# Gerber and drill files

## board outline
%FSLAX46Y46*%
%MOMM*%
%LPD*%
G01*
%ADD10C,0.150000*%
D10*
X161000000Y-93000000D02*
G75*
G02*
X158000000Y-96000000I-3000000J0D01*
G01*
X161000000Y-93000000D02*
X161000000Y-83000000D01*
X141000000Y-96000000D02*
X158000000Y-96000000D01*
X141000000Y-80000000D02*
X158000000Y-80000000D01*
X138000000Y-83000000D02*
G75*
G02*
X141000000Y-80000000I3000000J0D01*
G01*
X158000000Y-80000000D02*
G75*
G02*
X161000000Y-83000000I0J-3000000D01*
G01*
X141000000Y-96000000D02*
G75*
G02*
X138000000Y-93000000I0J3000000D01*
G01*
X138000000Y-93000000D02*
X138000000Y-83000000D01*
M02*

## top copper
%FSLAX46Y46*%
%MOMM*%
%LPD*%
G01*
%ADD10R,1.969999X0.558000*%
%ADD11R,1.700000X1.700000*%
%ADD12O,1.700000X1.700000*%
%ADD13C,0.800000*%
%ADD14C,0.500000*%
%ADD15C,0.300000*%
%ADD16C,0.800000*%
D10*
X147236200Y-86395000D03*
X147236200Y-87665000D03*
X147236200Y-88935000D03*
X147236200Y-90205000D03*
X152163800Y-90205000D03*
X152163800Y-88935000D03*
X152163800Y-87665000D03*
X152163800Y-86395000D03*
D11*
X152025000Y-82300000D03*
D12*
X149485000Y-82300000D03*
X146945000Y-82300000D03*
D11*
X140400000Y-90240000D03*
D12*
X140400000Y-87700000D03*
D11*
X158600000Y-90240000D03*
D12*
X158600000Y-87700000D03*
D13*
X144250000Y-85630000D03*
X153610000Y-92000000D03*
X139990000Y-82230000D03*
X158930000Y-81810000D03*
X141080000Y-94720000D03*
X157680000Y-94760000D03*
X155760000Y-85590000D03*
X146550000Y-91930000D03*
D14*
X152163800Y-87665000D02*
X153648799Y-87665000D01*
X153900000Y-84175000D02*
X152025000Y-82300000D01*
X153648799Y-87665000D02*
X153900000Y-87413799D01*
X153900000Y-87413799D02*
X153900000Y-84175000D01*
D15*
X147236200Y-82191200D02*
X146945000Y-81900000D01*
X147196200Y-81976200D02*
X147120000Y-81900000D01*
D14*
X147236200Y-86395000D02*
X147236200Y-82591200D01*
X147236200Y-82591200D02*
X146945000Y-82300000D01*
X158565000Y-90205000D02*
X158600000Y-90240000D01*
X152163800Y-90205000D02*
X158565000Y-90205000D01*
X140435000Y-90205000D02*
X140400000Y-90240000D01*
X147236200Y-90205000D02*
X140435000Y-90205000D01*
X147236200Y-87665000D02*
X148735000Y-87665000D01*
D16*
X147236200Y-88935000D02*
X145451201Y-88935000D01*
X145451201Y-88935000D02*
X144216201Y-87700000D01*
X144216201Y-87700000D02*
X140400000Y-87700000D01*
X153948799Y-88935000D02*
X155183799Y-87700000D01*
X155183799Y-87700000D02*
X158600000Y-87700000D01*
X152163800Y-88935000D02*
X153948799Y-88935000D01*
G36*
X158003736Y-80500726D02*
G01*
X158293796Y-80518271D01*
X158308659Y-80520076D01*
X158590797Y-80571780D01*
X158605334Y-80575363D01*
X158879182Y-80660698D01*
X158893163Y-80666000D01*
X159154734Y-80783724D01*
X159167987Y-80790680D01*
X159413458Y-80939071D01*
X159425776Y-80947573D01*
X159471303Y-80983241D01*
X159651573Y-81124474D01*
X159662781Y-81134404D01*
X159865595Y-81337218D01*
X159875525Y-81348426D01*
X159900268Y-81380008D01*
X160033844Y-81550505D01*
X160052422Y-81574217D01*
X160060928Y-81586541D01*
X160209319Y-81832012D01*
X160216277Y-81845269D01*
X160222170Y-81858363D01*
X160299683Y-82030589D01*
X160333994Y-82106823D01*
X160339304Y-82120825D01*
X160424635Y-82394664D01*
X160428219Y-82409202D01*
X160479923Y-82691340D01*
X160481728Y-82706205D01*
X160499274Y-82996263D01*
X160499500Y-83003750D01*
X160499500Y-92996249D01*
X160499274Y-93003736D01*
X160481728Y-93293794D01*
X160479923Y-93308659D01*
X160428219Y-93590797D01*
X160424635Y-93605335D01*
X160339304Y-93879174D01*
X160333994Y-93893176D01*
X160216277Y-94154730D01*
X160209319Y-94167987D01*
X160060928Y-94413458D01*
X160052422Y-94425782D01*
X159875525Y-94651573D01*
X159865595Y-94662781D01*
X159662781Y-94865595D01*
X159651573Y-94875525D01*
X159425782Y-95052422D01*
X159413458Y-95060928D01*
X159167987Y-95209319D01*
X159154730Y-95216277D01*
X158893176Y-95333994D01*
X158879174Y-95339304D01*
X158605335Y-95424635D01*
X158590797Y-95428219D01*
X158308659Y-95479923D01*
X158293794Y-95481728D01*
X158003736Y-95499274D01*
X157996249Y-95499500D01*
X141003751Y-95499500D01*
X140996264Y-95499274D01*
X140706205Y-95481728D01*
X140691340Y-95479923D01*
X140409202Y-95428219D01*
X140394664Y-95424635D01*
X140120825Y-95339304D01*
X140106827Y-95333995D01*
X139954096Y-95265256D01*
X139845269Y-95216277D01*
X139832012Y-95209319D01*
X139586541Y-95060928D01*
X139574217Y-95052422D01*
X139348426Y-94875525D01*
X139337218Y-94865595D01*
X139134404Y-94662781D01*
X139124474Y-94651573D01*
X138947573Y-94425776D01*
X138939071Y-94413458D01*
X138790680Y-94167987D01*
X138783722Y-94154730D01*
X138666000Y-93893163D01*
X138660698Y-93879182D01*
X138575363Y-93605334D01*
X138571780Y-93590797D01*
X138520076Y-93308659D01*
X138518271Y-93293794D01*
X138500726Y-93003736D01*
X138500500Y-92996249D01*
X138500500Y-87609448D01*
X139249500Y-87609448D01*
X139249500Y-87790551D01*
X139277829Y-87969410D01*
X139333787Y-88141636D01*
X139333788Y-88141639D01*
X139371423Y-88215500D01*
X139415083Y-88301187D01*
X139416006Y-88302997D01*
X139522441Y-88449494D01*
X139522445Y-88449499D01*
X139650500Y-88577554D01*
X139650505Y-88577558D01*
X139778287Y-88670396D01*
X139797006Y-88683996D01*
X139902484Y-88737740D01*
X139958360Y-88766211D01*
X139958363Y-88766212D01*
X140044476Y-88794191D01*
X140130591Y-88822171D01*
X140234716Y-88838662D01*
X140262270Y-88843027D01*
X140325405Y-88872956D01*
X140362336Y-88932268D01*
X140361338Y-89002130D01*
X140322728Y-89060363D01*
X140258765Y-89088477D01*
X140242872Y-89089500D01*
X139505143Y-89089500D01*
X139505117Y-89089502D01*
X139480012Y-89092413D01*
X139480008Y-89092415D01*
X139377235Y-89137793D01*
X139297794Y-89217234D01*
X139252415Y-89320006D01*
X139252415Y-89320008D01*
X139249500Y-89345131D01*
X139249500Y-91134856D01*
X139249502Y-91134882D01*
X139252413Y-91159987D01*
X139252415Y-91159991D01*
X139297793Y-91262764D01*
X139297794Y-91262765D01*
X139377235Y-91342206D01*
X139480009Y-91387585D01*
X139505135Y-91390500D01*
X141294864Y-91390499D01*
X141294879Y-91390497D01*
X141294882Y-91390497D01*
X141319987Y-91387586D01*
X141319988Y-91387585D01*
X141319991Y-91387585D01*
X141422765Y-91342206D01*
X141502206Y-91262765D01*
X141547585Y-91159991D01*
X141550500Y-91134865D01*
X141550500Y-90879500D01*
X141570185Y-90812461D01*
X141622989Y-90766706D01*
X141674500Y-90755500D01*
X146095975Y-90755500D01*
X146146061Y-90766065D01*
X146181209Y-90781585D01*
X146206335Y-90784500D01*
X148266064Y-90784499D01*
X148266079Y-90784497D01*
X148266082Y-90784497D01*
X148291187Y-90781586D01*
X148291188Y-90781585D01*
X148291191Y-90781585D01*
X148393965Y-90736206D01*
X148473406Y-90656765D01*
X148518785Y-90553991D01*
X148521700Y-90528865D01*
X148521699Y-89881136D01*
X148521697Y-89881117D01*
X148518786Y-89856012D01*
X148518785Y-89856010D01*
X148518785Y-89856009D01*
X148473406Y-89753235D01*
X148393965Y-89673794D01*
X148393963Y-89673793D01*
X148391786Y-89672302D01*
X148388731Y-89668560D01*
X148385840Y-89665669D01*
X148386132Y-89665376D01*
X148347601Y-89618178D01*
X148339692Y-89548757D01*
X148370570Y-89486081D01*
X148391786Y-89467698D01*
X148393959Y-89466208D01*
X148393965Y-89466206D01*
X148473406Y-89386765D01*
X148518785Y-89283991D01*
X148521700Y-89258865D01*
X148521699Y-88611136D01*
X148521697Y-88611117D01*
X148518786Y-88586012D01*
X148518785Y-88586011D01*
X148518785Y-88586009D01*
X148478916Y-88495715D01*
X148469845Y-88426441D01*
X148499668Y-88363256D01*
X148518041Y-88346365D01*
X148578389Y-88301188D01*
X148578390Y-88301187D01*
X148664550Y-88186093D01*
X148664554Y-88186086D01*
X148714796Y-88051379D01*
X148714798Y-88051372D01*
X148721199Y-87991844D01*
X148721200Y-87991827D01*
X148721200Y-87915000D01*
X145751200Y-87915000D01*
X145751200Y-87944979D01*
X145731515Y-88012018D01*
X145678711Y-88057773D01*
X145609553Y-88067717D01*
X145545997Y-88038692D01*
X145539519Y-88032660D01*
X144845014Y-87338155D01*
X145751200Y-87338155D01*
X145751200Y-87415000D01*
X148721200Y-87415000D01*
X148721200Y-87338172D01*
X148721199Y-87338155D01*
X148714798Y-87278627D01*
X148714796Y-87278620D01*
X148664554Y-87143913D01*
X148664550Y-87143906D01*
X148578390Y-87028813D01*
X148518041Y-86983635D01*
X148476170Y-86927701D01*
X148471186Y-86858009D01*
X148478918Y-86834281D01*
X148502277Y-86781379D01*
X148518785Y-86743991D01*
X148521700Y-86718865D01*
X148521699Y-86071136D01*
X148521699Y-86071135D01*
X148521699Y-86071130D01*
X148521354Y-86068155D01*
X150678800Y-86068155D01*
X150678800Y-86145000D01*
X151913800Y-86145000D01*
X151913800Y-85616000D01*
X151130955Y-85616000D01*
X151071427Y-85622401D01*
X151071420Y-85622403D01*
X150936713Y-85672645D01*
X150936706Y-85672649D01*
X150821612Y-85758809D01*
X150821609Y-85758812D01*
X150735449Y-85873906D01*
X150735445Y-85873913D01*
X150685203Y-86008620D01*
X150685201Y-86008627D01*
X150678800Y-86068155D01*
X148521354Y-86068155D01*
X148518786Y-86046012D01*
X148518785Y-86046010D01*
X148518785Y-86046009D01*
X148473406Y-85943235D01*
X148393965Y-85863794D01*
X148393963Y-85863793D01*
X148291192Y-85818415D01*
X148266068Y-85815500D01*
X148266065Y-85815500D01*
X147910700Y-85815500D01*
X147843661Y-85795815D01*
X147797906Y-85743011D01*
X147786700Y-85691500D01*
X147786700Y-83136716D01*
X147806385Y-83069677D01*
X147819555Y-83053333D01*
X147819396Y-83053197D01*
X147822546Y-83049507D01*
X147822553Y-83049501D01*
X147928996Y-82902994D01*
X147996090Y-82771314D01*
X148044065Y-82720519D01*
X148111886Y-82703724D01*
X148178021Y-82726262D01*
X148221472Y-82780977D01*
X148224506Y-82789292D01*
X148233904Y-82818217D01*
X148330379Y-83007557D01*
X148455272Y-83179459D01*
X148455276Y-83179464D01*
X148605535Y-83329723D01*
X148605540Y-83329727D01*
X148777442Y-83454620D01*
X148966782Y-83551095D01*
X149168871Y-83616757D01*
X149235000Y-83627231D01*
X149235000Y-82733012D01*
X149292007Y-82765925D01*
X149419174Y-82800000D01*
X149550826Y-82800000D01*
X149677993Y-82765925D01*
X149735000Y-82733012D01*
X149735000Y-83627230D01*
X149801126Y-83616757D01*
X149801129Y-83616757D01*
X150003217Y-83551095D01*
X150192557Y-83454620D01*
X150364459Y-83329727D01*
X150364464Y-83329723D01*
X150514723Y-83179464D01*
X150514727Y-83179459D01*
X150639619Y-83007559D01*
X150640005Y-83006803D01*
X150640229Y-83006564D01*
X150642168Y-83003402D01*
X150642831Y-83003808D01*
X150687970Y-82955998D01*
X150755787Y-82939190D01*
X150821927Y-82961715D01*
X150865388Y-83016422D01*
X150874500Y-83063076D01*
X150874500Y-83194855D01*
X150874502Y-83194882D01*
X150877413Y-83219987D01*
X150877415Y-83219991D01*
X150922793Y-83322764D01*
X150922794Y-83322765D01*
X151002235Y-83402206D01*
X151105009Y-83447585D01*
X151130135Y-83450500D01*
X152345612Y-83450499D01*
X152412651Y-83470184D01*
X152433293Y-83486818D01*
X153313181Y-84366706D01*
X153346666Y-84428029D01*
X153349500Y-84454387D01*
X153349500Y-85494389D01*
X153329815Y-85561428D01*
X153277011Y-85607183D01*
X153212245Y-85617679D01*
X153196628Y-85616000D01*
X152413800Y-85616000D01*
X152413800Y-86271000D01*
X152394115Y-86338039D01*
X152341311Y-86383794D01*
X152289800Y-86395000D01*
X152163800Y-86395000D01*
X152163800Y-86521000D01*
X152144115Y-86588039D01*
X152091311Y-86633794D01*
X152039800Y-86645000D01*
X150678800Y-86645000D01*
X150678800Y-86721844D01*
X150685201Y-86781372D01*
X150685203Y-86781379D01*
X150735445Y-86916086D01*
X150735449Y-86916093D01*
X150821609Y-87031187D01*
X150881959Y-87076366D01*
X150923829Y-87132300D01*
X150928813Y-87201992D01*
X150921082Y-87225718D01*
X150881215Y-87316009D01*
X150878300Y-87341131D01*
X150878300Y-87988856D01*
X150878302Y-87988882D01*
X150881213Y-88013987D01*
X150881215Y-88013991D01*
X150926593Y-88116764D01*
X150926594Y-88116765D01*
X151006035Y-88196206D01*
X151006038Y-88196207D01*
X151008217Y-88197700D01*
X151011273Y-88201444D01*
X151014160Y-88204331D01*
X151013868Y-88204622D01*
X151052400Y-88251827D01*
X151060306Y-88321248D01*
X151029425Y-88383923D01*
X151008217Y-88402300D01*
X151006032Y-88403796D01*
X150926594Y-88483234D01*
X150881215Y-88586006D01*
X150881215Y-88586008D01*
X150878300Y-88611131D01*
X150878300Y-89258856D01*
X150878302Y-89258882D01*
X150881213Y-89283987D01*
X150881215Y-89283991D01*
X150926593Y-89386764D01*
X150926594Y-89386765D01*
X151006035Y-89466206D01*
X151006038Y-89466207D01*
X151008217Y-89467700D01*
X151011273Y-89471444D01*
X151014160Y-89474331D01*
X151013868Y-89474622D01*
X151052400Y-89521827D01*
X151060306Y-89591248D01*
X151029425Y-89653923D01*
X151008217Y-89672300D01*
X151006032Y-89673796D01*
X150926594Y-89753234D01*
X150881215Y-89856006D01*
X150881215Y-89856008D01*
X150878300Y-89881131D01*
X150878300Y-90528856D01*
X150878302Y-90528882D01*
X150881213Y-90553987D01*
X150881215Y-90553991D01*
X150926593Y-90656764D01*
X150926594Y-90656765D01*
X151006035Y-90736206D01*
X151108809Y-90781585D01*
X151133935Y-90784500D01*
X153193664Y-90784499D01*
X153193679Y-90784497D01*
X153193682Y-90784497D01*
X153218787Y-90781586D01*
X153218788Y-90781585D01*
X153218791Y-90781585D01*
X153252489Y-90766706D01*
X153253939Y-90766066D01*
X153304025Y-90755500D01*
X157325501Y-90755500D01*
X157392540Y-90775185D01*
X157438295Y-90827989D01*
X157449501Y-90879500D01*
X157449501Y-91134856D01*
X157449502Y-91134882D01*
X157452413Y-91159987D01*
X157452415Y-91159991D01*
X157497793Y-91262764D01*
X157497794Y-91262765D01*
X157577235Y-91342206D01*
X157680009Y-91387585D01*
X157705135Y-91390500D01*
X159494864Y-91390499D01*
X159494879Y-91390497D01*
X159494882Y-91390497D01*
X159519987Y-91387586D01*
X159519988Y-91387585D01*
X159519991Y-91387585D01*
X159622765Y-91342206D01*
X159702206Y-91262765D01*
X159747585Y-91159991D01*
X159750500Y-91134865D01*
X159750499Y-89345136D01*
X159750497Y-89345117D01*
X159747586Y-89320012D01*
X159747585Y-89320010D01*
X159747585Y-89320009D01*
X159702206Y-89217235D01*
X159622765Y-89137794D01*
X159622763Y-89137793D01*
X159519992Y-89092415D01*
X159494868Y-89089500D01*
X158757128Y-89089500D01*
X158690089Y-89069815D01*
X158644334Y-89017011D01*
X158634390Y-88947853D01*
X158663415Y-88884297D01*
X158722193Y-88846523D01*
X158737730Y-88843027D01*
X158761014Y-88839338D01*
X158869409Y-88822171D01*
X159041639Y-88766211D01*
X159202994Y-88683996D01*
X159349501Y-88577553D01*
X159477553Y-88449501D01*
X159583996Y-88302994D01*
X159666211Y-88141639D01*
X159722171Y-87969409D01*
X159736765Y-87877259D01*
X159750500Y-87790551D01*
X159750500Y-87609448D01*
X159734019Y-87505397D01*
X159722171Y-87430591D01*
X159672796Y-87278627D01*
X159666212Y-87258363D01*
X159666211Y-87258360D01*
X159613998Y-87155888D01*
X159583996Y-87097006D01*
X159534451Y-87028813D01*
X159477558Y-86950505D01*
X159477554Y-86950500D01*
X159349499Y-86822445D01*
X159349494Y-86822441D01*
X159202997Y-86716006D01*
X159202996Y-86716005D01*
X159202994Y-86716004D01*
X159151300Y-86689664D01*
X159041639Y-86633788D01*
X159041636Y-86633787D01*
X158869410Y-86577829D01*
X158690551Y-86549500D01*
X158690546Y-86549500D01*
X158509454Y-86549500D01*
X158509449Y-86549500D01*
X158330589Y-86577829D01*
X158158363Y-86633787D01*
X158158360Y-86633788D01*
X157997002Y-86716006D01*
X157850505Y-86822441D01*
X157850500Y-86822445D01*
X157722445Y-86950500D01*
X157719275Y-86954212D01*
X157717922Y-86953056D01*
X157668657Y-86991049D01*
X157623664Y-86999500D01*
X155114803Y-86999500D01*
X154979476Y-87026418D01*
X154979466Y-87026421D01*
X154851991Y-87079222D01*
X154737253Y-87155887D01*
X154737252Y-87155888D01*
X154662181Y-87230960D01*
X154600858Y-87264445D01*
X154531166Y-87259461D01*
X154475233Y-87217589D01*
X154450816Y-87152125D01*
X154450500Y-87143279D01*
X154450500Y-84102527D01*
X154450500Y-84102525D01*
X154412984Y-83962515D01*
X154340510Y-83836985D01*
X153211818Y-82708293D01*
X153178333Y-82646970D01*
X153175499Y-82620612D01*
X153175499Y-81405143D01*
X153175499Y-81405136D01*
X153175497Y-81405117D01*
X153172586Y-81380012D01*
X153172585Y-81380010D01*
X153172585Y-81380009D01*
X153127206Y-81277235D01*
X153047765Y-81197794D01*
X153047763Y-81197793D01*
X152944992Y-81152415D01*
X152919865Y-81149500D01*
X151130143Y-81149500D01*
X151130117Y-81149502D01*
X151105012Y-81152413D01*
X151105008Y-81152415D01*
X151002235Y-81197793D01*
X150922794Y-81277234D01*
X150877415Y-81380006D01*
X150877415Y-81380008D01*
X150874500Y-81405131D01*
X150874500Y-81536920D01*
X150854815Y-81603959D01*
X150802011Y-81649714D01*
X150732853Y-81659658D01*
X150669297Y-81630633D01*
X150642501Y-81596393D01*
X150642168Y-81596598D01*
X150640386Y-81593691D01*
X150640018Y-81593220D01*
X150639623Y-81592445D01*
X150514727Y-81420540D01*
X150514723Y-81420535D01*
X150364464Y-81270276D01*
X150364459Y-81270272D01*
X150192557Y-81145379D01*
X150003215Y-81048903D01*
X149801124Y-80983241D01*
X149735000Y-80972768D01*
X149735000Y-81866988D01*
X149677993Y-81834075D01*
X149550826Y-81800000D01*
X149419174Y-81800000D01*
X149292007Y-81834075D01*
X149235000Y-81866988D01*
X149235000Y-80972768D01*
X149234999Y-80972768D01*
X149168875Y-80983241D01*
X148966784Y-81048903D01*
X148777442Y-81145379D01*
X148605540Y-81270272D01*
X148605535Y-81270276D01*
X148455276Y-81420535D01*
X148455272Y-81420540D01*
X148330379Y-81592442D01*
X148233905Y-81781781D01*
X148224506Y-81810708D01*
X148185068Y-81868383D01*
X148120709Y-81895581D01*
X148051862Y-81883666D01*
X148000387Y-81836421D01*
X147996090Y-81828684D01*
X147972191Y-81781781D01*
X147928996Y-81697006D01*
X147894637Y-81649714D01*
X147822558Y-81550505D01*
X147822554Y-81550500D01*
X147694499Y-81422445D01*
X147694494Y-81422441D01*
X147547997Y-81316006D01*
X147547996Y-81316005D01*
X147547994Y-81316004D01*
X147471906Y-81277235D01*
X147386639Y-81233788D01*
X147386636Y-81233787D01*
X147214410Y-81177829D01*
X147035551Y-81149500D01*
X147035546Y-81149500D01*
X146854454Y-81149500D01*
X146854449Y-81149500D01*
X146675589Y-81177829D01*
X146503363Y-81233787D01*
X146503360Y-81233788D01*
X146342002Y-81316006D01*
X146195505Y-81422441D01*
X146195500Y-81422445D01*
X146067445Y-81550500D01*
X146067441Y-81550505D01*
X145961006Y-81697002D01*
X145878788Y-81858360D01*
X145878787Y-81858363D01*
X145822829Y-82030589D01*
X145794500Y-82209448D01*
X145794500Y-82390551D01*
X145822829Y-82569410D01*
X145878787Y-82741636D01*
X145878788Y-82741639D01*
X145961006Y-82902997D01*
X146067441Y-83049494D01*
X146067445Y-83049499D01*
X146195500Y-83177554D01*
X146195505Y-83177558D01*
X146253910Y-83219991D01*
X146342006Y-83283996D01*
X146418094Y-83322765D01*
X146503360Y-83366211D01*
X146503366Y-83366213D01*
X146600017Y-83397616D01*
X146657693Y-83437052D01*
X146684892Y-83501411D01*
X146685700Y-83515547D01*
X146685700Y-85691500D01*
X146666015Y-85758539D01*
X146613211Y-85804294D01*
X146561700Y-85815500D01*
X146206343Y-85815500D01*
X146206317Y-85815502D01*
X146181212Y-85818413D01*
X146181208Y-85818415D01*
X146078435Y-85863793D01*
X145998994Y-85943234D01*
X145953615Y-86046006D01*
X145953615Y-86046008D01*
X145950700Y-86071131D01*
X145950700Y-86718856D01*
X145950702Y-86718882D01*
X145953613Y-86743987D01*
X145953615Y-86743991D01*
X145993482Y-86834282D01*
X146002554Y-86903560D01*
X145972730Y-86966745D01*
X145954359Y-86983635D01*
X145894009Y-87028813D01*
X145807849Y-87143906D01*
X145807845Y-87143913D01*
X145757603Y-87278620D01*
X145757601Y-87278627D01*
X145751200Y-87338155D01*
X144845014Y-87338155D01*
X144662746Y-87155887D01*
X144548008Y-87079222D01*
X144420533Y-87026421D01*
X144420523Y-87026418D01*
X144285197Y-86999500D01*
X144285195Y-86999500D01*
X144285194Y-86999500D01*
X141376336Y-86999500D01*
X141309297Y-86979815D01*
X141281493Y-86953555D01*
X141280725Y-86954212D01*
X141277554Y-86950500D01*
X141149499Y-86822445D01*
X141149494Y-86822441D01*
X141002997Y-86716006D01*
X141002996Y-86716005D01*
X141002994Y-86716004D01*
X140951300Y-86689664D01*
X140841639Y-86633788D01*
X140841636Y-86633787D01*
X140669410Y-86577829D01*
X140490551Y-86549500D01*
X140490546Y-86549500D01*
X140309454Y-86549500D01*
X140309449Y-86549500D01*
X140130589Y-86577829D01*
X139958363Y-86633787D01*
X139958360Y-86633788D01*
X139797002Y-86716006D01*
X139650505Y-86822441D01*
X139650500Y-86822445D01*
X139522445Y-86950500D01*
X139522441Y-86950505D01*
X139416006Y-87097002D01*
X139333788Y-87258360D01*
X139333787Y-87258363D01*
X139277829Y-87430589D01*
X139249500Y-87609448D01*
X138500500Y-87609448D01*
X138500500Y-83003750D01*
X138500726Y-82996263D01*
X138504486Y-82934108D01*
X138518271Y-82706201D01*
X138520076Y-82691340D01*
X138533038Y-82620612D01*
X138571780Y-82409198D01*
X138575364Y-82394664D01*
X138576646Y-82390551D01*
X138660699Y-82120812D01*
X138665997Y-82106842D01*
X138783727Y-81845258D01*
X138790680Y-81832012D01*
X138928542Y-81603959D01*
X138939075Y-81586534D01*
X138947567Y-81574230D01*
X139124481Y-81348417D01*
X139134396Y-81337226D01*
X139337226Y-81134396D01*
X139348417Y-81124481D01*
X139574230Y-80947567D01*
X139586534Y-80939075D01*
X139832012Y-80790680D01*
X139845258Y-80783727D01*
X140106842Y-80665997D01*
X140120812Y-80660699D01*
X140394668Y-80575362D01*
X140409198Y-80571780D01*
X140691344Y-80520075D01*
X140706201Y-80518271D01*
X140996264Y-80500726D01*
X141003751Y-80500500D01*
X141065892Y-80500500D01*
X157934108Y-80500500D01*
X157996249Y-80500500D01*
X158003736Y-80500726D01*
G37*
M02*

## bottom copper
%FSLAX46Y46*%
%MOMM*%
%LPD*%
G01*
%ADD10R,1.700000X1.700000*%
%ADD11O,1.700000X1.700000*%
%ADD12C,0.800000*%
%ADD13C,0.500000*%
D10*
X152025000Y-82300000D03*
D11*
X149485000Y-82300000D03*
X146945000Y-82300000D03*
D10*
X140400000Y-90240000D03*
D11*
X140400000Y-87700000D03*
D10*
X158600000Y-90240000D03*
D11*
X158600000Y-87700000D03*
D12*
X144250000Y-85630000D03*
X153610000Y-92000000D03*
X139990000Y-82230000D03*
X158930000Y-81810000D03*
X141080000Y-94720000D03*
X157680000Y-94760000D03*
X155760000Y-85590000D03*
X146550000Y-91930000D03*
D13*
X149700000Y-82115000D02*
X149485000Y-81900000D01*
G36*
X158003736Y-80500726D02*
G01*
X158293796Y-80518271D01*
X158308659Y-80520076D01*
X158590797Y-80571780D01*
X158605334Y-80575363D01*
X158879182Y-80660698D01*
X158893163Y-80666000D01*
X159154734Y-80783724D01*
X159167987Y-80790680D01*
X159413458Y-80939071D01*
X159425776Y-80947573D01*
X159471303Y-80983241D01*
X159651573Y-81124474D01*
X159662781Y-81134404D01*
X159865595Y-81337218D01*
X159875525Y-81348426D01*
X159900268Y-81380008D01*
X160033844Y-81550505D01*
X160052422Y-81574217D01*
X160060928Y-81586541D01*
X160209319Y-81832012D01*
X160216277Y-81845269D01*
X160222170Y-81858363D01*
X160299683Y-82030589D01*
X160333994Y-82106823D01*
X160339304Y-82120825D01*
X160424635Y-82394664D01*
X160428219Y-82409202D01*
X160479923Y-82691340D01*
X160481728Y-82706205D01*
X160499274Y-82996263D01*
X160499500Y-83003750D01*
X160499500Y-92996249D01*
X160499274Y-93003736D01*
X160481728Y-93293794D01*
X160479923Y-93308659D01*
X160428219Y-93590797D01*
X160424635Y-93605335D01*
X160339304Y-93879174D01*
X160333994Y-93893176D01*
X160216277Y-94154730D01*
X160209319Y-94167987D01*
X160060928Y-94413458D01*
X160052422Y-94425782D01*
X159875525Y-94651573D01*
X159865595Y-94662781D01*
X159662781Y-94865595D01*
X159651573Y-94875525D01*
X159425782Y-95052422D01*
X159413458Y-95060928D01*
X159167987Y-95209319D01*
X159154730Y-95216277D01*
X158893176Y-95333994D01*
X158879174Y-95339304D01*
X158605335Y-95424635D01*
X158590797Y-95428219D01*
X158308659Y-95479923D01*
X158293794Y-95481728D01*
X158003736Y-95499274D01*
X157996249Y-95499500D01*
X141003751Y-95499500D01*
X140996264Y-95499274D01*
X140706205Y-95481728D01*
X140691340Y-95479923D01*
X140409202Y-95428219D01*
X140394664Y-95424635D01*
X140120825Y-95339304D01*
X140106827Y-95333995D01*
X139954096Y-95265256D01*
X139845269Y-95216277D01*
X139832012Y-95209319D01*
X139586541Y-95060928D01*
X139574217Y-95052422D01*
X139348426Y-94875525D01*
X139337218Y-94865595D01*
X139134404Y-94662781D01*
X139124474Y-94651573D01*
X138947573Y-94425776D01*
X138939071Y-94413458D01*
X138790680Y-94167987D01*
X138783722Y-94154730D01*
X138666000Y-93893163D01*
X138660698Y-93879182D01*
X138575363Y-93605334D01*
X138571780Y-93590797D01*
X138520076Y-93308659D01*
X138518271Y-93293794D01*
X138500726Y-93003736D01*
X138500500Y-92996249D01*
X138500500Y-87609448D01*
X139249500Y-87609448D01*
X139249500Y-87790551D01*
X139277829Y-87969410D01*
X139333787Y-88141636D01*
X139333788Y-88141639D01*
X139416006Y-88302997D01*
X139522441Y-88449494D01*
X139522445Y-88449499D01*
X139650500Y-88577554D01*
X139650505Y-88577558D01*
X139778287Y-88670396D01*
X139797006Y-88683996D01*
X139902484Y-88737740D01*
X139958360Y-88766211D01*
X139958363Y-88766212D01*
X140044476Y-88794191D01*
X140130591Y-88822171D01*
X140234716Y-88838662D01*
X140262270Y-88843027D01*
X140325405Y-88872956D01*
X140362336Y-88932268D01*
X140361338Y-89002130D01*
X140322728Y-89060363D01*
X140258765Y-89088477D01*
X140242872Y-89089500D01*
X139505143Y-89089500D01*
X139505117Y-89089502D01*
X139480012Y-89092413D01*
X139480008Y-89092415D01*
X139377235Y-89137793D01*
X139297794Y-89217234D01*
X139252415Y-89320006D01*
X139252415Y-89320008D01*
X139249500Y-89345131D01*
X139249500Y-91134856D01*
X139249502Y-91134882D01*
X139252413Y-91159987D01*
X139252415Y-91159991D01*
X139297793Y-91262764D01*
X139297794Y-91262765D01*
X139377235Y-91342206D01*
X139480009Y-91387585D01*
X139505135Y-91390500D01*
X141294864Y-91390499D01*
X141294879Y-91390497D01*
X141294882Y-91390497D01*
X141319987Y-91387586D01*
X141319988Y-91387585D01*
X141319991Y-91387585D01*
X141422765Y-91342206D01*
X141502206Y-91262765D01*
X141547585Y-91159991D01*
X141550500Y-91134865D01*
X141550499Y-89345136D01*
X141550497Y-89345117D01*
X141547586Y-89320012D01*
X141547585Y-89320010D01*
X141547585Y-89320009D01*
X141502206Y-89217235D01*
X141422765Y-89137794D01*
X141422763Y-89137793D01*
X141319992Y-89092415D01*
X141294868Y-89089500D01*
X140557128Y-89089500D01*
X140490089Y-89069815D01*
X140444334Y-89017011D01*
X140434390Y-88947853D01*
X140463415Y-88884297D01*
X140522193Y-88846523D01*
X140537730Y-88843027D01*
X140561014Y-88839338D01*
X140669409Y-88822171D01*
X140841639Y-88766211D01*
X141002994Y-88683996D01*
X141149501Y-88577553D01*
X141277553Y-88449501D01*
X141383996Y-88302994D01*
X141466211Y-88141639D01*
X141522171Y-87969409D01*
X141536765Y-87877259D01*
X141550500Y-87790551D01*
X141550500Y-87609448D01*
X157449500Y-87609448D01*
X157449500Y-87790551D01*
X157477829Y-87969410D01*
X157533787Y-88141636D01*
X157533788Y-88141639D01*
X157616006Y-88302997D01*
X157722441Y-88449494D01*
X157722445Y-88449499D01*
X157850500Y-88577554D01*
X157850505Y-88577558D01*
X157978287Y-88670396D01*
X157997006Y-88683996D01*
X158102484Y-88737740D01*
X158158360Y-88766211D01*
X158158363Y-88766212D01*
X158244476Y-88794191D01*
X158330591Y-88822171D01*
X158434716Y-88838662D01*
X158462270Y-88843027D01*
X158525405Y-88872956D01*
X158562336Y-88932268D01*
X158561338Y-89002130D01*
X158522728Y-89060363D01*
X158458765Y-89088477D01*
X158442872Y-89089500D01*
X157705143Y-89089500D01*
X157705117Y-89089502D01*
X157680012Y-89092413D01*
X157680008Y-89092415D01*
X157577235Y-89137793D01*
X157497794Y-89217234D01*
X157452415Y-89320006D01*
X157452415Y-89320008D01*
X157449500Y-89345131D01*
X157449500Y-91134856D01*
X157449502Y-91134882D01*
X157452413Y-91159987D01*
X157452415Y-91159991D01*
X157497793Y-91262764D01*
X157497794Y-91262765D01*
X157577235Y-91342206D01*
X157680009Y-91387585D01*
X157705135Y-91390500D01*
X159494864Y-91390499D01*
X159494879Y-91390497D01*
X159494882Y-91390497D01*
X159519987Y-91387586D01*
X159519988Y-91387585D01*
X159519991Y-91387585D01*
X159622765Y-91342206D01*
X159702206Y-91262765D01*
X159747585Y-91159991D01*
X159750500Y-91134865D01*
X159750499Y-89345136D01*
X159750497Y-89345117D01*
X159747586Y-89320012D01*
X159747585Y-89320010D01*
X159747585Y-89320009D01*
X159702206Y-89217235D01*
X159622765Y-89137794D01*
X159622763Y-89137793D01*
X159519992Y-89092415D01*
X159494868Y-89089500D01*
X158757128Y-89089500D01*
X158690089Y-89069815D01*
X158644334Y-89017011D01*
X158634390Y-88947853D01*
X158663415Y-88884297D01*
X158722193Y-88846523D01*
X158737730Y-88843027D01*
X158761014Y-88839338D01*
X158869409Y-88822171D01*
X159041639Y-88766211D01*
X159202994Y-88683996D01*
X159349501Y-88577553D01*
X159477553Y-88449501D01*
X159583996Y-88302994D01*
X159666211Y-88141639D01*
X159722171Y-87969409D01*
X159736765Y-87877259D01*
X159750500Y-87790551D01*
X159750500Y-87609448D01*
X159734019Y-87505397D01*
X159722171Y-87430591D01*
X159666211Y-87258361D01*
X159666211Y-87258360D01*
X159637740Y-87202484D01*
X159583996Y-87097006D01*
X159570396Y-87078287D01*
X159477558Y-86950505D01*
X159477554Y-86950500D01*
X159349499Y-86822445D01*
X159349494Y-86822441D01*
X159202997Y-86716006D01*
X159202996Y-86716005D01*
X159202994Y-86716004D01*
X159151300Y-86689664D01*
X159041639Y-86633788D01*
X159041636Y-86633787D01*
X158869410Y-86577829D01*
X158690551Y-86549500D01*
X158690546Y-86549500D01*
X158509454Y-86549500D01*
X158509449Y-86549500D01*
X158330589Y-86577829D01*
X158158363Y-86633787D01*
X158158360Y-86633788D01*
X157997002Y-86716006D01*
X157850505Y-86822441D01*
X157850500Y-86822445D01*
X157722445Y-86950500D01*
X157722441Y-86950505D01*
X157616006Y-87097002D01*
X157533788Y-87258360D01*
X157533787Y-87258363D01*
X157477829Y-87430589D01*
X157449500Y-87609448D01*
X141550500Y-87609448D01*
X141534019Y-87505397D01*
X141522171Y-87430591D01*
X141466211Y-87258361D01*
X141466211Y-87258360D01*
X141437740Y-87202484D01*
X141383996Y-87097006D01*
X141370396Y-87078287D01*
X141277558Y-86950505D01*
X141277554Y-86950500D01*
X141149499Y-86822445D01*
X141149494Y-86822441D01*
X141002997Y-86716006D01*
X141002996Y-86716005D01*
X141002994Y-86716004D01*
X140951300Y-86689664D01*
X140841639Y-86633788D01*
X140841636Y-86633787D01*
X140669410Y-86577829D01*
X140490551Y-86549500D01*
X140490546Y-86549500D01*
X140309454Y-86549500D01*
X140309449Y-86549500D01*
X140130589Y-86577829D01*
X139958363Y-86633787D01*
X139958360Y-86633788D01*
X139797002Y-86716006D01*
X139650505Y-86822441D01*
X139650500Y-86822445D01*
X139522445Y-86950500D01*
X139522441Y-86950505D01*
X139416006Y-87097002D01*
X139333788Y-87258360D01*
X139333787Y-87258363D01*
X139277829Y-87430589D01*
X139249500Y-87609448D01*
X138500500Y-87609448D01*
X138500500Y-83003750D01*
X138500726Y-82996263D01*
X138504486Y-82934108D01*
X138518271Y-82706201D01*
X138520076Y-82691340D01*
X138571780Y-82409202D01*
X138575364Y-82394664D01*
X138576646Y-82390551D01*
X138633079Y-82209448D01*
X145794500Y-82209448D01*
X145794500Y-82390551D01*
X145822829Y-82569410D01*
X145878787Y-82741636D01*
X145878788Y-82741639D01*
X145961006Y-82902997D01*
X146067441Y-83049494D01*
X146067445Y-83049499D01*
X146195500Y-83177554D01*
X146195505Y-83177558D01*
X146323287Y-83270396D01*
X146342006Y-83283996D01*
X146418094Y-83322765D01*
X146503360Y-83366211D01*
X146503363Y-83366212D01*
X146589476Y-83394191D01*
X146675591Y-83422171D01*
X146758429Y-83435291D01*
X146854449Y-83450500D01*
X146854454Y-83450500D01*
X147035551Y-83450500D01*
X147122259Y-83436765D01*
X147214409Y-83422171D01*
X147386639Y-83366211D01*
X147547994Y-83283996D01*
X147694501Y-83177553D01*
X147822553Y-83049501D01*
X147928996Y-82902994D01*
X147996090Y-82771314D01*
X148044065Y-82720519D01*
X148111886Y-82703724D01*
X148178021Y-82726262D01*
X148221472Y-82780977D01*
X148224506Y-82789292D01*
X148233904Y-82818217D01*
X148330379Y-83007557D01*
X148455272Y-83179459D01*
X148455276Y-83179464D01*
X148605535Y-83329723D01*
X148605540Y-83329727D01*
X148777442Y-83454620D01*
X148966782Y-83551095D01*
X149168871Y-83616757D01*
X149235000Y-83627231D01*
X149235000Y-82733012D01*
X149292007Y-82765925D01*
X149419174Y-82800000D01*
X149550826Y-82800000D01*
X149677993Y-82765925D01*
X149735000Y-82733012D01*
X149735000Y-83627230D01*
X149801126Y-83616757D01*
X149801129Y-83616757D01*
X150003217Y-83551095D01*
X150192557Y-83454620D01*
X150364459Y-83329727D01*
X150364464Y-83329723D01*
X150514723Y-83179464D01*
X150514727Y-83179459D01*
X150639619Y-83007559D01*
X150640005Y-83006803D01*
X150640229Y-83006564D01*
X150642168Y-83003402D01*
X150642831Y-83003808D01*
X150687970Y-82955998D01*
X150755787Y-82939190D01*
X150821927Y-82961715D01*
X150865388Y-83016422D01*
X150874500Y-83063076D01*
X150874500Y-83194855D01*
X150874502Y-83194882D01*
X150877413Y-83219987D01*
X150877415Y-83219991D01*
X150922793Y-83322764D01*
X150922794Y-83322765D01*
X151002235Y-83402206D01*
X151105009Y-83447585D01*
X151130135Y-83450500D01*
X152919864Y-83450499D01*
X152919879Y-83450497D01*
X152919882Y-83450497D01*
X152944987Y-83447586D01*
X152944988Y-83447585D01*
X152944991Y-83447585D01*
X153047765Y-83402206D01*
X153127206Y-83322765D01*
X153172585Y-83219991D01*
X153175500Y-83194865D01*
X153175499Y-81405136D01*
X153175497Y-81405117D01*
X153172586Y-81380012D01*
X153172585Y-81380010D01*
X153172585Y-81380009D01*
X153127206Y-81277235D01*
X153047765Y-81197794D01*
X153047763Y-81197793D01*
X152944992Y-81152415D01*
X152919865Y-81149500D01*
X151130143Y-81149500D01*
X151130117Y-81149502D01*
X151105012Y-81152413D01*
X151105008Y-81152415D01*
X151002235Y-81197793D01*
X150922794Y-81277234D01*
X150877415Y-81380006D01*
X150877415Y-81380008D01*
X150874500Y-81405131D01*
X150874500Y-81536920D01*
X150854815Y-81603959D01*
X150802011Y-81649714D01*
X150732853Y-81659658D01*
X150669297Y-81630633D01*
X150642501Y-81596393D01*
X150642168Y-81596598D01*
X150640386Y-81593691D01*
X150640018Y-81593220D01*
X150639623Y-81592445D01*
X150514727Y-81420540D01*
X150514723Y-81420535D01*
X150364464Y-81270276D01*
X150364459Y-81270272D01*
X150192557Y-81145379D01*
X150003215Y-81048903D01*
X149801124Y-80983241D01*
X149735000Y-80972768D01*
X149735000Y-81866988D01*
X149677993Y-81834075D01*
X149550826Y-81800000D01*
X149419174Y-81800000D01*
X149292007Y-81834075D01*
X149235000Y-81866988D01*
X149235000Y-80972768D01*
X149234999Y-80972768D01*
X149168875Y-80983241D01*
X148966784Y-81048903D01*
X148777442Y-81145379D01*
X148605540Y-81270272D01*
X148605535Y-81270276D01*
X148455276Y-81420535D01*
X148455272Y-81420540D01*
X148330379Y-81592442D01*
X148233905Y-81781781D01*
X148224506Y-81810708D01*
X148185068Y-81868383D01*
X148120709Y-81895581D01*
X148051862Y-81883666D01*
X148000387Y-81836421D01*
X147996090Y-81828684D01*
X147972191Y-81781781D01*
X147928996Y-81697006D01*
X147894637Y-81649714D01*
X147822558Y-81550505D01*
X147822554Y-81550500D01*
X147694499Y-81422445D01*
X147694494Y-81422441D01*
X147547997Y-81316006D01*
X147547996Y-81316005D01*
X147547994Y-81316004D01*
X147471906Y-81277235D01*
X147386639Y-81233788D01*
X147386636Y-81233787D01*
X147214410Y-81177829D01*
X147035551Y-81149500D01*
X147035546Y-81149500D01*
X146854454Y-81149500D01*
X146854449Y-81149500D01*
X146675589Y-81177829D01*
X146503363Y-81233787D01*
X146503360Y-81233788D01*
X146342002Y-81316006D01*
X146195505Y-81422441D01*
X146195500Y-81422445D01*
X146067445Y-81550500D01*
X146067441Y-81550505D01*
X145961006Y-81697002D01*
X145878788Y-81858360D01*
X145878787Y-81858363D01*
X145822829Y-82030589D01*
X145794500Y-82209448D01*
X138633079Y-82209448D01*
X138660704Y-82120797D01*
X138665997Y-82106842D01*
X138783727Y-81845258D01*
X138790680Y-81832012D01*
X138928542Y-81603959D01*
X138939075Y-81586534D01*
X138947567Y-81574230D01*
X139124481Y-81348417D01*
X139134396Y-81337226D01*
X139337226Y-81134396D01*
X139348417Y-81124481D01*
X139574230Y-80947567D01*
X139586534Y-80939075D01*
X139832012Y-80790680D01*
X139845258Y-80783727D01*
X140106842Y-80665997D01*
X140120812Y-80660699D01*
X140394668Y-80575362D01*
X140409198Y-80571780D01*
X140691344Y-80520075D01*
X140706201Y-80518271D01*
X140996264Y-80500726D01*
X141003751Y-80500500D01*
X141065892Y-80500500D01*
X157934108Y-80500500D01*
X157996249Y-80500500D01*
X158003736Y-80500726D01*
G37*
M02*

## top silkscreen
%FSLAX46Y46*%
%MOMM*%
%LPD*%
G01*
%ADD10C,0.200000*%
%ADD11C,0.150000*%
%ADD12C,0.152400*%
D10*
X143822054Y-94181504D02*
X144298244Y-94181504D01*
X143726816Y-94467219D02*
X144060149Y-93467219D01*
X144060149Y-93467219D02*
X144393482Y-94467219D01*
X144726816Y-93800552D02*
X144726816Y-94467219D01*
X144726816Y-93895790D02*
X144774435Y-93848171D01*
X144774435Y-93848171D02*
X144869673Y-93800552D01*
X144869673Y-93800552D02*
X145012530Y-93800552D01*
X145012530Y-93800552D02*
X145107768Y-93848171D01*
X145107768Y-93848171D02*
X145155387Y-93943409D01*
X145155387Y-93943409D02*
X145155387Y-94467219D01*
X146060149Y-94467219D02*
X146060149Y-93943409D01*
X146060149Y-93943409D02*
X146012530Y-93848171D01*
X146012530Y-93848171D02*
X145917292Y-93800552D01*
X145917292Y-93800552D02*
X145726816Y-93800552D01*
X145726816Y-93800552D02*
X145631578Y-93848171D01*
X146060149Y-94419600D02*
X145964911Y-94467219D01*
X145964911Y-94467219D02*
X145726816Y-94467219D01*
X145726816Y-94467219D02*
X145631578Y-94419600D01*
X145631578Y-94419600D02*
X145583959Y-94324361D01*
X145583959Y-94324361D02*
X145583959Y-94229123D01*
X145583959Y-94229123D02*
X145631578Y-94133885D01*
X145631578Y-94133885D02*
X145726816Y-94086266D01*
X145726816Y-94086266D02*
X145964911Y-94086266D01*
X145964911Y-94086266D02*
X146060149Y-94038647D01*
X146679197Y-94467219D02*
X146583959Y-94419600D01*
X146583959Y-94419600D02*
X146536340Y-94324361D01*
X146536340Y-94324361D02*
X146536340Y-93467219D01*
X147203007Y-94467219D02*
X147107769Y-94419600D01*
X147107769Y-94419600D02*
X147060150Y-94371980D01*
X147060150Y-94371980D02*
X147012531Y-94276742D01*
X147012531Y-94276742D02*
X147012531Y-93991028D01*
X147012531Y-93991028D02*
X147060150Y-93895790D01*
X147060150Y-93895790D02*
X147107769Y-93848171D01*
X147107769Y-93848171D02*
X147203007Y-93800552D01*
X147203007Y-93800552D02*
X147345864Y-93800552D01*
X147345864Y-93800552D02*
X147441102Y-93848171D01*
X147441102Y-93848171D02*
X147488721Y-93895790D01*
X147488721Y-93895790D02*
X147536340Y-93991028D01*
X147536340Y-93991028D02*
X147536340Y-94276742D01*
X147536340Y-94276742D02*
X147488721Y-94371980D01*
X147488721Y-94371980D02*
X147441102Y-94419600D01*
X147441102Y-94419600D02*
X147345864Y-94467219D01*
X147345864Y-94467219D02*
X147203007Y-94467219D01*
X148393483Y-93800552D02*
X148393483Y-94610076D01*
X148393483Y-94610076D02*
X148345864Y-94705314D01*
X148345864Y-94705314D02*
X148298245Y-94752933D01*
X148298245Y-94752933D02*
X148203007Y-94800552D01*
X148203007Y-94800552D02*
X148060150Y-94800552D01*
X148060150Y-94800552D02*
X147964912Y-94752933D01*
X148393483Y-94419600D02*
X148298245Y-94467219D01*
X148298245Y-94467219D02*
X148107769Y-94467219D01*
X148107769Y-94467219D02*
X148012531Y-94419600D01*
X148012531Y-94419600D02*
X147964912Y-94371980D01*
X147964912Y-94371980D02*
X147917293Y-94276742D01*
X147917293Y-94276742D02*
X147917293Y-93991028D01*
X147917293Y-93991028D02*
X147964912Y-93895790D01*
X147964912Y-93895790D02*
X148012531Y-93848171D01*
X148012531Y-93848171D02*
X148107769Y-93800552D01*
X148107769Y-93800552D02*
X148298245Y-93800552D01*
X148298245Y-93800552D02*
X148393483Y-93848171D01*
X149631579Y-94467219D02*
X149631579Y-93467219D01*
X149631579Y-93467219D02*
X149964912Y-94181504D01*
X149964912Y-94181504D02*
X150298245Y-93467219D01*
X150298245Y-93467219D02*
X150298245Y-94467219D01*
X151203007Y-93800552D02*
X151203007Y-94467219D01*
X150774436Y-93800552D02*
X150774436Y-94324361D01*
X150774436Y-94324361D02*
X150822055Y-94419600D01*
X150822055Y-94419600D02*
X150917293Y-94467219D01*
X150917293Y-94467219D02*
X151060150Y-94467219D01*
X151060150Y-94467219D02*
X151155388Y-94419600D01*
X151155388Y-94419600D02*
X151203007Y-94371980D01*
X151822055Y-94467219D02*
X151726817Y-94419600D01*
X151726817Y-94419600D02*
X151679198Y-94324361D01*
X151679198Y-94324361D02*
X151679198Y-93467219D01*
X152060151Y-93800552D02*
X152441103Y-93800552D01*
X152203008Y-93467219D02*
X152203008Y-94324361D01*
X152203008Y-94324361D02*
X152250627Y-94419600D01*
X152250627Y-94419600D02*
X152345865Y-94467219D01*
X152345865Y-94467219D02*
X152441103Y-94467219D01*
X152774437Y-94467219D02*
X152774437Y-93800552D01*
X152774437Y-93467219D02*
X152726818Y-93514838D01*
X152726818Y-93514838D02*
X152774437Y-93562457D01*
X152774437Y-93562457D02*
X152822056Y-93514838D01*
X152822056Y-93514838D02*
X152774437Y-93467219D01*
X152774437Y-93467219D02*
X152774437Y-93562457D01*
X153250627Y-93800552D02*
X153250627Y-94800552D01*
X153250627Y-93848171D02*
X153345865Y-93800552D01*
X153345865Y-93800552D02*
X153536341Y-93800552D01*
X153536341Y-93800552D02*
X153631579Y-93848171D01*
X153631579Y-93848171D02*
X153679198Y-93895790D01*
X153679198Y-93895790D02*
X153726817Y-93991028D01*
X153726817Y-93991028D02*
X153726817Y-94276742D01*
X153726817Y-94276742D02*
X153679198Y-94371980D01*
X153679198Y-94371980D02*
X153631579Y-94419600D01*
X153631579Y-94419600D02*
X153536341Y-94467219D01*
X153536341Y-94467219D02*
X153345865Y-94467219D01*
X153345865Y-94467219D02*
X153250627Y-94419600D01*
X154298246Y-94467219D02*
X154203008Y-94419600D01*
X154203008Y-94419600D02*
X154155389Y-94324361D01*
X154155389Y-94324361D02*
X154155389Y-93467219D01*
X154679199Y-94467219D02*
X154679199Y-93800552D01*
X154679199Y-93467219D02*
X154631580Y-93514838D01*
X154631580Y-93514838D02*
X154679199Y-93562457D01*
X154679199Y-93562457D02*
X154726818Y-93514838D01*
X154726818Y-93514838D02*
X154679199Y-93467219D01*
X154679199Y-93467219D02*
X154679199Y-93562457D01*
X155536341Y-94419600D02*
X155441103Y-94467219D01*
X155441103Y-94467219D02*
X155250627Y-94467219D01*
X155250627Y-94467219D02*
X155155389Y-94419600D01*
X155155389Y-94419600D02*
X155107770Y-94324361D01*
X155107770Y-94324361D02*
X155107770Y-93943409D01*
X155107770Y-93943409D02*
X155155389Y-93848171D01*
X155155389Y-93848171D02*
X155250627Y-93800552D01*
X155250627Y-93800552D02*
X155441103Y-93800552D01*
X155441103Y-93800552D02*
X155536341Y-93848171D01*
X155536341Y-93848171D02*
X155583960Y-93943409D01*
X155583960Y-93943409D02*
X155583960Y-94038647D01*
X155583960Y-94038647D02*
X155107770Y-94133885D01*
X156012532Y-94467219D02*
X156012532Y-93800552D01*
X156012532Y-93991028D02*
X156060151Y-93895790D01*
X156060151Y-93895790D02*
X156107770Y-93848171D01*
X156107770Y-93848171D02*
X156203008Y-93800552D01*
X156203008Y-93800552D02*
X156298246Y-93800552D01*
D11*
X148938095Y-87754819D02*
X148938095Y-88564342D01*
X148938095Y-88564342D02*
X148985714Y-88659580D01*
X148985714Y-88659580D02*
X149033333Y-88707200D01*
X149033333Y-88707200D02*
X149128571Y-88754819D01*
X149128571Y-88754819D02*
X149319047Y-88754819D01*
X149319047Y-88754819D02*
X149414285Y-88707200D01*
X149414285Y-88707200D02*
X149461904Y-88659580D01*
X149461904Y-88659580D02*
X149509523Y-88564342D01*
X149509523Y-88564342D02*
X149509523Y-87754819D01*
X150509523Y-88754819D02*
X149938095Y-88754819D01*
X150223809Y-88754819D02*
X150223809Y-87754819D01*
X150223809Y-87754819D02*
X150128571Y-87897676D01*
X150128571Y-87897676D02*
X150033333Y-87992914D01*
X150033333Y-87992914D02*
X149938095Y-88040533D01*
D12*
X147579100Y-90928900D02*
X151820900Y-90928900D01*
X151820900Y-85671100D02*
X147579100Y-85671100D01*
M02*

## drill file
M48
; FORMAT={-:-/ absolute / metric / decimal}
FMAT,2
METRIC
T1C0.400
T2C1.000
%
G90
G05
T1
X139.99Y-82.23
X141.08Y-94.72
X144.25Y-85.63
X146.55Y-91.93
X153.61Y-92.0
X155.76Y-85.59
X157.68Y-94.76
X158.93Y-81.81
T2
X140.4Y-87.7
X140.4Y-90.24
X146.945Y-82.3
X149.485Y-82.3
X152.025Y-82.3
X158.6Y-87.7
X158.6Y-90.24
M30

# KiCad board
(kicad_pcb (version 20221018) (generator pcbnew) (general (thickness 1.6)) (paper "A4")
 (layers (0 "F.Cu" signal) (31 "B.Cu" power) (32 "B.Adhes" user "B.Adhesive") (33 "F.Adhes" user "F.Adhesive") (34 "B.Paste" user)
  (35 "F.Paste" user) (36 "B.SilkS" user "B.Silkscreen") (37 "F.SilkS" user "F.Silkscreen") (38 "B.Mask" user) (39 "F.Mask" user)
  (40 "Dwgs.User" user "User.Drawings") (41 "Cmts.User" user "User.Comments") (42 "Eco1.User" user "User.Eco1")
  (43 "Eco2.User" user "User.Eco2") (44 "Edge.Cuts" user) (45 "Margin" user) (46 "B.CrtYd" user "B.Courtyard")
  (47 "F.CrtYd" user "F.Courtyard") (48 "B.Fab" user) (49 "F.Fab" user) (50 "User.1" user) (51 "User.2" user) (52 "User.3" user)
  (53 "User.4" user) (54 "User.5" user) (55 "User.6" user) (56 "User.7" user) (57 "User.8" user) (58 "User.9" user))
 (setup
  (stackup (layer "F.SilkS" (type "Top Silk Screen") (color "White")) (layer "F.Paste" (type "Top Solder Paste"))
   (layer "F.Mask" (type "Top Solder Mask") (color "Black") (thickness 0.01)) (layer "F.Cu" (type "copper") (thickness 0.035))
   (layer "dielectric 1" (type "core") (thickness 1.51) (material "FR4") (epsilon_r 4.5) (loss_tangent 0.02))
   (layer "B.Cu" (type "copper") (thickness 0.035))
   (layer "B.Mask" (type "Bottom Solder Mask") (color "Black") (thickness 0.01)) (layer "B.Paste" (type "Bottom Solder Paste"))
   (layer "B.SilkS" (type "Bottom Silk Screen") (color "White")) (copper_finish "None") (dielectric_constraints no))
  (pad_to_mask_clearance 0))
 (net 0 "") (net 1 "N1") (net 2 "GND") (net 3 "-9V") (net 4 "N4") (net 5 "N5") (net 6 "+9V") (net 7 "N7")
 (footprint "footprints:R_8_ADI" (layer "F.Cu") (at 149.7 88.3)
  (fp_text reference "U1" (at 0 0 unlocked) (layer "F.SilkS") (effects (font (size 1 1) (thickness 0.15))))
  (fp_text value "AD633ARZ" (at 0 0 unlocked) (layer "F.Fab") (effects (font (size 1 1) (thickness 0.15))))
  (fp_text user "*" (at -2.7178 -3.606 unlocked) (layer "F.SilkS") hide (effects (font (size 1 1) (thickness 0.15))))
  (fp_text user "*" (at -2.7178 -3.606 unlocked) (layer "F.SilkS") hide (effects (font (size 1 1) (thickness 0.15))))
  (fp_line (start -2.1209 2.6289) (end 2.1209 2.6289) (stroke (width 0.1524) (type solid)) (layer "F.SilkS"))
  (fp_line (start 2.1209 -2.6289) (end -2.1209 -2.6289) (stroke (width 0.1524) (type solid)) (layer "F.SilkS"))
  (pad "1" smd rect (at -2.4638 -1.905) (size 1.969999 0.558) (layers "F.Cu" "F.Paste" "F.Mask") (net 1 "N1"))
  (pad "2" smd rect (at -2.4638 -0.635) (size 1.969999 0.558) (layers "F.Cu" "F.Paste" "F.Mask") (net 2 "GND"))
  (pad "3" smd rect (at -2.4638 0.635) (size 1.969999 0.558) (layers "F.Cu" "F.Paste" "F.Mask") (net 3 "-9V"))
  (pad "4" smd rect (at -2.4638 1.905) (size 1.969999 0.558) (layers "F.Cu" "F.Paste" "F.Mask") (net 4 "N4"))
  (pad "5" smd rect (at 2.4638 1.905) (size 1.969999 0.558) (layers "F.Cu" "F.Paste" "F.Mask") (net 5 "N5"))
  (pad "6" smd rect (at 2.4638 0.635) (size 1.969999 0.558) (layers "F.Cu" "F.Paste" "F.Mask") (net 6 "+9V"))
  (pad "7" smd rect (at 2.4638 -0.635) (size 1.969999 0.558) (layers "F.Cu" "F.Paste" "F.Mask") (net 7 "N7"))
  (pad "8" smd rect (at 2.4638 -1.905) (size 1.969999 0.558) (layers "F.Cu" "F.Paste" "F.Mask") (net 2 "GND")))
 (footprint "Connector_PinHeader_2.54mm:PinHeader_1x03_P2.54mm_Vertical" (layer "B.Cu") (at 152.025 82.3 90)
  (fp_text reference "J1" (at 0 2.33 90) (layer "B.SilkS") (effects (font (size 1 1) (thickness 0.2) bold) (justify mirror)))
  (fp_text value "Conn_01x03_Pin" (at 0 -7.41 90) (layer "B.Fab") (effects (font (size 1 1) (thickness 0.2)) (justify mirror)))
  (pad "1" thru_hole rect (at 0 0 90) (size 1.7 1.7) (drill 1) (layers "*.Cu" "*.Mask") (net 7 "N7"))
  (pad "2" thru_hole oval (at 0 -2.54 90) (size 1.7 1.7) (drill 1) (layers "*.Cu" "*.Mask") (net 2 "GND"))
  (pad "3" thru_hole oval (at 0 -5.08 90) (size 1.7 1.7) (drill 1) (layers "*.Cu" "*.Mask") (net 1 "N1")))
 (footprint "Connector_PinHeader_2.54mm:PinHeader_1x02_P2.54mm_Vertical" (layer "B.Cu") (at 140.4 90.24)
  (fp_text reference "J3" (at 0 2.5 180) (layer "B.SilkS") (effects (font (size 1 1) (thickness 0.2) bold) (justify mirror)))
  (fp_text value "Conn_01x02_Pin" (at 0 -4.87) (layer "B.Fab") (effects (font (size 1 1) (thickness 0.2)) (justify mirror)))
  (pad "1" thru_hole rect (at 0 0) (size 1.7 1.7) (drill 1) (layers "*.Cu" "*.Mask") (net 4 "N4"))
  (pad "2" thru_hole oval (at 0 -2.54) (size 1.7 1.7) (drill 1) (layers "*.Cu" "*.Mask") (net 3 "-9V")))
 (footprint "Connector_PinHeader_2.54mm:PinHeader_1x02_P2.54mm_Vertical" (layer "B.Cu") (at 158.6 90.24)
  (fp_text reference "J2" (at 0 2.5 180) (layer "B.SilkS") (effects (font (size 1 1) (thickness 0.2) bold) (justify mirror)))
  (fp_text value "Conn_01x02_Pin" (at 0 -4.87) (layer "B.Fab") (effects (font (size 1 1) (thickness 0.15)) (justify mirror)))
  (pad "1" thru_hole rect (at 0 0) (size 1.7 1.7) (drill 1) (layers "*.Cu" "*.Mask") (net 5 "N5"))
  (pad "2" thru_hole oval (at 0 -2.54) (size 1.7 1.7) (drill 1) (layers "*.Cu" "*.Mask") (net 6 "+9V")))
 (gr_arc (start 161 93) (mid 160.12132 95.12132) (end 158 96) (stroke (width 0.15) (type default)) (layer "Edge.Cuts"))
 (gr_line (start 161 93) (end 161 83) (stroke (width 0.15) (type default)) (layer "Edge.Cuts"))
 (gr_line (start 141 96) (end 158 96) (stroke (width 0.15) (type default)) (layer "Edge.Cuts"))
 (gr_line (start 141 80) (end 158 80) (stroke (width 0.15) (type default)) (layer "Edge.Cuts"))
 (gr_arc (start 138 83) (mid 138.87868 80.87868) (end 141 80) (stroke (width 0.15) (type default)) (layer "Edge.Cuts"))
 (gr_arc (start 158 80) (mid 160.12132 80.87868) (end 161 83) (stroke (width 0.15) (type default)) (layer "Edge.Cuts"))
 (gr_arc (start 141 96) (mid 138.87868 95.12132) (end 138 93) (stroke (width 0.15) (type default)) (layer "Edge.Cuts"))
 (gr_line (start 138 93) (end 138 83) (stroke (width 0.15) (type default)) (layer "Edge.Cuts"))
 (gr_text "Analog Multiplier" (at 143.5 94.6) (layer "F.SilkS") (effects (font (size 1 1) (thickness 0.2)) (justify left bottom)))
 (segment (start 152.1638 87.665) (end 153.648799 87.665) (width 0.5) (layer "F.Cu") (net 7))
 (segment (start 153.9 84.175) (end 152.025 82.3) (width 0.5) (layer "F.Cu") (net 7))
 (segment (start 153.648799 87.665) (end 153.9 87.413799) (width 0.5) (layer "F.Cu") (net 7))
 (segment (start 153.9 87.413799) (end 153.9 84.175) (width 0.5) (layer "F.Cu") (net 7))
 (segment (start 147.2362 82.1912) (end 146.945 81.9) (width 0.3) (layer "F.Cu") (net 1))
 (segment (start 147.1962 81.9762) (end 147.12 81.9) (width 0.3) (layer "F.Cu") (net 1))
 (segment (start 147.2362 86.395) (end 147.2362 82.5912) (width 0.5) (layer "F.Cu") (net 1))
 (segment (start 147.2362 82.5912) (end 146.945 82.3) (width 0.5) (layer "F.Cu") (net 1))
 (segment (start 158.565 90.205) (end 158.6 90.24) (width 0.5) (layer "F.Cu") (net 5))
 (segment (start 152.1638 90.205) (end 158.565 90.205) (width 0.5) (layer "F.Cu") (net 5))
 (segment (start 140.435 90.205) (end 140.4 90.24) (width 0.5) (layer "F.Cu") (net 4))
 (segment (start 147.2362 90.205) (end 140.435 90.205) (width 0.5) (layer "F.Cu") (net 4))
 (segment (start 147.2362 87.665) (end 148.735 87.665) (width 0.5) (layer "F.Cu") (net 2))
 (via (at 144.25 85.63) (size 0.8) (drill 0.4) (layers "F.Cu" "B.Cu") (free) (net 2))
 (via (at 153.61 92) (size 0.8) (drill 0.4) (layers "F.Cu" "B.Cu") (free) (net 2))
 (via (at 139.99 82.23) (size 0.8) (drill 0.4) (layers "F.Cu" "B.Cu") (free) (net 2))
 (via (at 158.93 81.81) (size 0.8) (drill 0.4) (layers "F.Cu" "B.Cu") (free) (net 2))
 (via (at 141.08 94.72) (size 0.8) (drill 0.4) (layers "F.Cu" "B.Cu") (free) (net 2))
 (via (at 157.68 94.76) (size 0.8) (drill 0.4) (layers "F.Cu" "B.Cu") (free) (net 2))
 (via (at 155.76 85.59) (size 0.8) (drill 0.4) (layers "F.Cu" "B.Cu") (free) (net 2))
 (via (at 146.55 91.93) (size 0.8) (drill 0.4) (layers "F.Cu" "B.Cu") (free) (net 2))
 (segment (start 149.7 82.115) (end 149.485 81.9) (width 0.5) (layer "B.Cu") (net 2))
 (segment (start 147.2362 88.935) (end 145.451201 88.935) (width 0.8) (layer "F.Cu") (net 3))
 (segment (start 145.451201 88.935) (end 144.216201 87.7) (width 0.8) (layer "F.Cu") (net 3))
 (segment (start 144.216201 87.7) (end 140.4 87.7) (width 0.8) (layer "F.Cu") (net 3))
 (segment (start 153.948799 88.935) (end 155.183799 87.7) (width 0.8) (layer "F.Cu") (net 6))
 (segment (start 155.183799 87.7) (end 158.6 87.7) (width 0.8) (layer "F.Cu") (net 6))
 (segment (start 152.1638 88.935) (end 153.948799 88.935) (width 0.8) (layer "F.Cu") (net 6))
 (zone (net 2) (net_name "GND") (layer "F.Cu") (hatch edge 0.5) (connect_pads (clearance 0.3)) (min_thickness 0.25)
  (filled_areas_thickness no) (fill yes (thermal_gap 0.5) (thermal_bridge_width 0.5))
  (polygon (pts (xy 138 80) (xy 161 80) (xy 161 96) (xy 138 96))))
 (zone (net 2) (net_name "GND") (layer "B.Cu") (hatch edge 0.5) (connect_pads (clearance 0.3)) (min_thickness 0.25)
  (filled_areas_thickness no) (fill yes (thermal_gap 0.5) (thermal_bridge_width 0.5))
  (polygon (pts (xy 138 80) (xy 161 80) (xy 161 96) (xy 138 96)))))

